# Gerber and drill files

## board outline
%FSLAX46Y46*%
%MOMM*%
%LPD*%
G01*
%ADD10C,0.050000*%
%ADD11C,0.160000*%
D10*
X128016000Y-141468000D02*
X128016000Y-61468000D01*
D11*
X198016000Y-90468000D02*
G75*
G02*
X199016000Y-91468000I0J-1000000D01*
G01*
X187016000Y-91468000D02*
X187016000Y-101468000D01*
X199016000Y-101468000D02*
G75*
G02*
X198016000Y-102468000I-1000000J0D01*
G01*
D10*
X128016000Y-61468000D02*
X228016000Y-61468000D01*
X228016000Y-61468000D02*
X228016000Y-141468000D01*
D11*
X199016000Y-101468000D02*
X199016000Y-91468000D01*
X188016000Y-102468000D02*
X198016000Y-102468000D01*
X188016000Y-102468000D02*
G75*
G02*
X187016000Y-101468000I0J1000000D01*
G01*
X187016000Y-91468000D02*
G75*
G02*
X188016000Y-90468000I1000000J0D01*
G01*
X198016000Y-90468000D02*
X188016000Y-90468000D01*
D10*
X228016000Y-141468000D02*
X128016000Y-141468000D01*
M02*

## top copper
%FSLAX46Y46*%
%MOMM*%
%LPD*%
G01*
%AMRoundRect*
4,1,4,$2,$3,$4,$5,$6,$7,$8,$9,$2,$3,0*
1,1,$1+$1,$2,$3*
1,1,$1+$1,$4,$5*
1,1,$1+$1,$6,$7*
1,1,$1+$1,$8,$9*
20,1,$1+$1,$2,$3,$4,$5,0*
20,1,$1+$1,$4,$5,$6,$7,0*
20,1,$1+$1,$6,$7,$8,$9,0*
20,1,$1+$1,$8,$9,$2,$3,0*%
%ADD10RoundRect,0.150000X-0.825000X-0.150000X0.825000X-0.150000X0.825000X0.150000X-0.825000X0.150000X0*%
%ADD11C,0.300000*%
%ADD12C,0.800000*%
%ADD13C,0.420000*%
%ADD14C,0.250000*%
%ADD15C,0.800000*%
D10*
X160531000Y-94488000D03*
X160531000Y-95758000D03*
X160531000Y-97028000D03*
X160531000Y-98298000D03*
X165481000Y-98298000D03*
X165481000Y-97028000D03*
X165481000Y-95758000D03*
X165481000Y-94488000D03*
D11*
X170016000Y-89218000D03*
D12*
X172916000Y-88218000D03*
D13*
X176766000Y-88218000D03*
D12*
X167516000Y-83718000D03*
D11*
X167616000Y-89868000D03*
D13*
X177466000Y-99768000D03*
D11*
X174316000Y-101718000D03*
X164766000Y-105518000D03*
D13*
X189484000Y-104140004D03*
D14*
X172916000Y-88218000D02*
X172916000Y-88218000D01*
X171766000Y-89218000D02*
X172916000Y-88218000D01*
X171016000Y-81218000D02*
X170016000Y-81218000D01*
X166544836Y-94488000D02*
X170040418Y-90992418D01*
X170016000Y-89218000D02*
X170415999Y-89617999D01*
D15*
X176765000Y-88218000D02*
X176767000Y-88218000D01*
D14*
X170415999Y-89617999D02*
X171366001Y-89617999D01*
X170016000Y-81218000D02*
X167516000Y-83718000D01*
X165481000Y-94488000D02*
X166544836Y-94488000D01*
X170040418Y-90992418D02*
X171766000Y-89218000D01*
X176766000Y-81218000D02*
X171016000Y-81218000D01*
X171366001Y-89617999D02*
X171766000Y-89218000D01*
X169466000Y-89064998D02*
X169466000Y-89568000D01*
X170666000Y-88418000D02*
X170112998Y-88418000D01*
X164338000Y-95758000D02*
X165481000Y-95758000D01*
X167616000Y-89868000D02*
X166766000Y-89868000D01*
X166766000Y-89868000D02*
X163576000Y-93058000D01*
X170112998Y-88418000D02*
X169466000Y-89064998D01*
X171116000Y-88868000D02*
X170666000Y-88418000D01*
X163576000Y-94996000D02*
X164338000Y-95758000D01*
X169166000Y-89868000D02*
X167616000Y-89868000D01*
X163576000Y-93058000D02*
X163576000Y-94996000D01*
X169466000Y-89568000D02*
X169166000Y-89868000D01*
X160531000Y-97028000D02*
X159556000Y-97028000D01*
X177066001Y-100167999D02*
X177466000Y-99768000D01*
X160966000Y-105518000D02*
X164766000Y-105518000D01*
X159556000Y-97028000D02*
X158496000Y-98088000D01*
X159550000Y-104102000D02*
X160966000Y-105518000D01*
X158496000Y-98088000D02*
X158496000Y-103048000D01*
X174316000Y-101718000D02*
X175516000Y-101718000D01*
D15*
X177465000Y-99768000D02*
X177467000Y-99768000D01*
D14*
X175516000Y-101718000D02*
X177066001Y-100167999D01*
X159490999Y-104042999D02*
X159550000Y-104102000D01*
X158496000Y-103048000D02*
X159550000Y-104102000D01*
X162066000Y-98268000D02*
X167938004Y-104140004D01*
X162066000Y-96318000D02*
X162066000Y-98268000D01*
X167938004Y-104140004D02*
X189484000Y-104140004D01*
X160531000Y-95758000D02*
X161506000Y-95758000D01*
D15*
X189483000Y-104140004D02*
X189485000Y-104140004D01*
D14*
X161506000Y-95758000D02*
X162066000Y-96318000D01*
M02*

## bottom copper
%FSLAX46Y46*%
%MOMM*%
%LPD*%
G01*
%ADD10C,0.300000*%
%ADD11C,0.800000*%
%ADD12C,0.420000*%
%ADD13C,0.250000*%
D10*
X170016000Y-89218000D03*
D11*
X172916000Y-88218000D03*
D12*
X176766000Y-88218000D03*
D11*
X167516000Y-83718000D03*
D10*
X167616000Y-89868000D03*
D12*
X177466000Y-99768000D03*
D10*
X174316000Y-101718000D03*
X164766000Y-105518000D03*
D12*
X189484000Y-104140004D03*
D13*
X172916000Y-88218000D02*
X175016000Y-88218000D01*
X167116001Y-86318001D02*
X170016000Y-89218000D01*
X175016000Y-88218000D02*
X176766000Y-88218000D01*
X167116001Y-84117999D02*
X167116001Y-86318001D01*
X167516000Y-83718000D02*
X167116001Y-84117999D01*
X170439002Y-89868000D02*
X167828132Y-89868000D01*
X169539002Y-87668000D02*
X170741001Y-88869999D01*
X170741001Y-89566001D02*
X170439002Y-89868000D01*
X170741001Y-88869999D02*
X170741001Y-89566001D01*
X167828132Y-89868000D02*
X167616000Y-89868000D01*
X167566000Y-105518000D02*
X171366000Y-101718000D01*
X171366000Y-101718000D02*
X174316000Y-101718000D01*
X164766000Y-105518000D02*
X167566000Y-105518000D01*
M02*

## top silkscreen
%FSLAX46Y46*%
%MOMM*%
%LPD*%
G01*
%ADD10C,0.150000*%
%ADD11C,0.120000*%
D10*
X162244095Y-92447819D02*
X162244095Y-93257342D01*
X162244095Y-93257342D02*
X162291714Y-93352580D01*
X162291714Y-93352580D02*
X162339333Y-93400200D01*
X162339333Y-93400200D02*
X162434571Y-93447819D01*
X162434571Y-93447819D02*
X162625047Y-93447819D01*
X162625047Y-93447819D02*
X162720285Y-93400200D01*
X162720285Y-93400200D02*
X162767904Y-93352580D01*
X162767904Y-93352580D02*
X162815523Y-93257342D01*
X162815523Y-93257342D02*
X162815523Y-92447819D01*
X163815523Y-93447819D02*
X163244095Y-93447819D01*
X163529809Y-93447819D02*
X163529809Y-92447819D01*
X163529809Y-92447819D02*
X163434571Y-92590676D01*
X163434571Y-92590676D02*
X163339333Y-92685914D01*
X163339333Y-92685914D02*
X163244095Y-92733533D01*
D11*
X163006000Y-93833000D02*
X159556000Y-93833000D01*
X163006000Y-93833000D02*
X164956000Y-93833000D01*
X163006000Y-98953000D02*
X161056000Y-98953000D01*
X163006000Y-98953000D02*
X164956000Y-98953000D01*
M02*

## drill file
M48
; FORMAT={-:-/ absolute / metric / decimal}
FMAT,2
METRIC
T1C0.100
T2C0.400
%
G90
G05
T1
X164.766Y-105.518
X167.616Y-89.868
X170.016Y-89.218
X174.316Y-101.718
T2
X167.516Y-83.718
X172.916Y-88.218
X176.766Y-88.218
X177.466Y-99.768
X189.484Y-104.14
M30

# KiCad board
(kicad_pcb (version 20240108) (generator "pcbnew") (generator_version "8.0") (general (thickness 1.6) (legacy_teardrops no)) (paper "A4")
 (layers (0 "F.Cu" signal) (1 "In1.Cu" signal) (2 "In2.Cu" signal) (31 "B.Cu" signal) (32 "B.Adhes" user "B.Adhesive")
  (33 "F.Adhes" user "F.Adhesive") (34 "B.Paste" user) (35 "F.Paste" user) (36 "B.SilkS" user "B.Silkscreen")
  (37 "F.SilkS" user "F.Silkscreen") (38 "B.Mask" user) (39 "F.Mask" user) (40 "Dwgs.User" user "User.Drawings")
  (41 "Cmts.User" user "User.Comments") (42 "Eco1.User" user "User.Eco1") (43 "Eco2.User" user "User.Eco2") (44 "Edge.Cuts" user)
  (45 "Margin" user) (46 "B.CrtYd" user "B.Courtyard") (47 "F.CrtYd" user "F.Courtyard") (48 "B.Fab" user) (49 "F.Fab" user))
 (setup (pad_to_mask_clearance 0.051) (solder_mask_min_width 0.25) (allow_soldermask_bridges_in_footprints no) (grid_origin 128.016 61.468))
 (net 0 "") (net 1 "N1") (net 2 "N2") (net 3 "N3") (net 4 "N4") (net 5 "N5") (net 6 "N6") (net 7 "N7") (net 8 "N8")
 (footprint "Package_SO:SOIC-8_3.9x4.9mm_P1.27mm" (layer "F.Cu") (at 163.006 96.393)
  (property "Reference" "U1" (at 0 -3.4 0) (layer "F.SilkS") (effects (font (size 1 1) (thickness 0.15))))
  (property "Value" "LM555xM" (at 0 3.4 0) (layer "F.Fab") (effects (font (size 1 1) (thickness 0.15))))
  (fp_line (start 0 -2.56) (end -3.45 -2.56) (stroke (width 0.12) (type solid)) (layer "F.SilkS"))
  (fp_line (start 0 -2.56) (end 1.95 -2.56) (stroke (width 0.12) (type solid)) (layer "F.SilkS"))
  (fp_line (start 0 2.56) (end -1.95 2.56) (stroke (width 0.12) (type solid)) (layer "F.SilkS"))
  (fp_line (start 0 2.56) (end 1.95 2.56) (stroke (width 0.12) (type solid)) (layer "F.SilkS"))
  (pad "1" smd roundrect (at -2.475 -1.905) (size 1.95 0.6) (layers "F.Cu" "F.Paste" "F.Mask") (roundrect_rratio 0.25) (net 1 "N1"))
  (pad "2" smd roundrect (at -2.475 -0.635) (size 1.95 0.6) (layers "F.Cu" "F.Paste" "F.Mask") (roundrect_rratio 0.25) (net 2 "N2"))
  (pad "3" smd roundrect (at -2.475 0.635) (size 1.95 0.6) (layers "F.Cu" "F.Paste" "F.Mask") (roundrect_rratio 0.25) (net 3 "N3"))
  (pad "4" smd roundrect (at -2.475 1.905) (size 1.95 0.6) (layers "F.Cu" "F.Paste" "F.Mask") (roundrect_rratio 0.25) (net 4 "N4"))
  (pad "5" smd roundrect (at 2.475 1.905) (size 1.95 0.6) (layers "F.Cu" "F.Paste" "F.Mask") (roundrect_rratio 0.25) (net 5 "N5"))
  (pad "6" smd roundrect (at 2.475 0.635) (size 1.95 0.6) (layers "F.Cu" "F.Paste" "F.Mask") (roundrect_rratio 0.25) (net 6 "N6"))
  (pad "7" smd roundrect (at 2.475 -0.635) (size 1.95 0.6) (layers "F.Cu" "F.Paste" "F.Mask") (roundrect_rratio 0.25) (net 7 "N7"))
  (pad "8" smd roundrect (at 2.475 -1.905) (size 1.95 0.6) (layers "F.Cu" "F.Paste" "F.Mask") (roundrect_rratio 0.25) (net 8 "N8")))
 (gr_line (start 128.016 141.468) (end 128.016 61.468) (stroke (width 0.05) (type solid)) (layer "Edge.Cuts"))
 (gr_arc (start 198.016 90.468) (mid 198.723107 90.760893) (end 199.016 91.468) (stroke (width 0.16) (type solid)) (layer "Edge.Cuts"))
 (gr_line (start 187.016 91.468) (end 187.016 101.468) (stroke (width 0.16) (type solid)) (layer "Edge.Cuts"))
 (gr_arc (start 199.016 101.468) (mid 198.723107 102.175107) (end 198.016 102.468) (stroke (width 0.16) (type solid)) (layer "Edge.Cuts"))
 (gr_line (start 128.016 61.468) (end 228.016 61.468) (stroke (width 0.05) (type solid)) (layer "Edge.Cuts"))
 (gr_line (start 228.016 61.468) (end 228.016 141.468) (stroke (width 0.05) (type solid)) (layer "Edge.Cuts"))
 (gr_line (start 199.016 101.468) (end 199.016 91.468) (stroke (width 0.16) (type solid)) (layer "Edge.Cuts"))
 (gr_line (start 188.016 102.468) (end 198.016 102.468) (stroke (width 0.16) (type solid)) (layer "Edge.Cuts"))
 (gr_arc (start 188.016 102.468) (mid 187.308893 102.175107) (end 187.016 101.468) (stroke (width 0.16) (type solid)) (layer "Edge.Cuts"))
 (gr_arc (start 187.016 91.468) (mid 187.308893 90.760893) (end 188.016 90.468) (stroke (width 0.16) (type solid)) (layer "Edge.Cuts"))
 (gr_line (start 198.016 90.468) (end 188.016 90.468) (stroke (width 0.16) (type solid)) (layer "Edge.Cuts"))
 (gr_line (start 228.016 141.468) (end 128.016 141.468) (stroke (width 0.05) (type solid)) (layer "Edge.Cuts"))
 (segment (start 172.916 88.218) (end 172.916 88.218) (width 0.25) (layer "F.Cu") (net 8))
 (segment (start 171.766 89.218) (end 172.916 88.218) (width 0.25) (layer "F.Cu") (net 8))
 (segment (start 171.016 81.218) (end 170.016 81.218) (width 0.25) (layer "F.Cu") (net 8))
 (segment (start 166.544836 94.488) (end 170.040418 90.992418) (width 0.25) (layer "F.Cu") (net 8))
 (segment (start 170.016 89.218) (end 170.415999 89.617999) (width 0.25) (layer "F.Cu") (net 8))
 (segment (start 176.765 88.218) (end 176.767 88.218) (width 0.8) (layer "F.Cu") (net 8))
 (segment (start 170.415999 89.617999) (end 171.366001 89.617999) (width 0.25) (layer "F.Cu") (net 8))
 (segment (start 170.016 81.218) (end 167.516 83.718) (width 0.25) (layer "F.Cu") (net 8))
 (segment (start 165.481 94.488) (end 166.544836 94.488) (width 0.25) (layer "F.Cu") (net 8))
 (segment (start 170.040418 90.992418) (end 171.766 89.218) (width 0.25) (layer "F.Cu") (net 8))
 (segment (start 176.766 81.218) (end 171.016 81.218) (width 0.25) (layer "F.Cu") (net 8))
 (segment (start 171.366001 89.617999) (end 171.766 89.218) (width 0.25) (layer "F.Cu") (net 8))
 (via (at 170.016 89.218) (size 0.3) (drill 0.1) (layers "F.Cu" "B.Cu") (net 8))
 (via (at 172.916 88.218) (size 0.8) (drill 0.4) (layers "F.Cu" "B.Cu") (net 8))
 (via (at 176.766 88.218) (size 0.42) (drill 0.4) (layers "F.Cu" "B.Cu") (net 8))
 (via (at 167.516 83.718) (size 0.8) (drill 0.4) (layers "F.Cu" "B.Cu") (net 8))
 (segment (start 172.916 88.218) (end 175.016 88.218) (width 0.25) (layer "B.Cu") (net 8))
 (segment (start 167.116001 86.318001) (end 170.016 89.218) (width 0.25) (layer "B.Cu") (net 8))
 (segment (start 175.016 88.218) (end 176.766 88.218) (width 0.25) (layer "B.Cu") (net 8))
 (segment (start 167.116001 84.117999) (end 167.116001 86.318001) (width 0.25) (layer "B.Cu") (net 8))
 (segment (start 167.516 83.718) (end 167.116001 84.117999) (width 0.25) (layer "B.Cu") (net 8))
 (segment (start 169.466 89.064998) (end 169.466 89.568) (width 0.25) (layer "F.Cu") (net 7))
 (segment (start 170.666 88.418) (end 170.112998 88.418) (width 0.25) (layer "F.Cu") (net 7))
 (segment (start 164.338 95.758) (end 165.481 95.758) (width 0.25) (layer "F.Cu") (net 7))
 (segment (start 167.616 89.868) (end 166.766 89.868) (width 0.25) (layer "F.Cu") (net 7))
 (segment (start 166.766 89.868) (end 163.576 93.058) (width 0.25) (layer "F.Cu") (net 7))
 (segment (start 170.112998 88.418) (end 169.466 89.064998) (width 0.25) (layer "F.Cu") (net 7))
 (segment (start 171.116 88.868) (end 170.666 88.418) (width 0.25) (layer "F.Cu") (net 7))
 (segment (start 163.576 94.996) (end 164.338 95.758) (width 0.25) (layer "F.Cu") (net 7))
 (segment (start 169.166 89.868) (end 167.616 89.868) (width 0.25) (layer "F.Cu") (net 7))
 (segment (start 163.576 93.058) (end 163.576 94.996) (width 0.25) (layer "F.Cu") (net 7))
 (segment (start 169.466 89.568) (end 169.166 89.868) (width 0.25) (layer "F.Cu") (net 7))
 (via (at 167.616 89.868) (size 0.3) (drill 0.1) (layers "F.Cu" "B.Cu") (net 7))
 (segment (start 170.439002 89.868) (end 167.828132 89.868) (width 0.25) (layer "B.Cu") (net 7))
 (segment (start 169.539002 87.668) (end 170.741001 88.869999) (width 0.25) (layer "B.Cu") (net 7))
 (segment (start 170.741001 89.566001) (end 170.439002 89.868) (width 0.25) (layer "B.Cu") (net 7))
 (segment (start 170.741001 88.869999) (end 170.741001 89.566001) (width 0.25) (layer "B.Cu") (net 7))
 (segment (start 167.828132 89.868) (end 167.616 89.868) (width 0.25) (layer "B.Cu") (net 7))
 (segment (start 160.531 97.028) (end 159.556 97.028) (width 0.25) (layer "F.Cu") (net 3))
 (segment (start 177.066001 100.167999) (end 177.466 99.768) (width 0.25) (layer "F.Cu") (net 3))
 (segment (start 160.966 105.518) (end 164.766 105.518) (width 0.25) (layer "F.Cu") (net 3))
 (segment (start 159.556 97.028) (end 158.496 98.088) (width 0.25) (layer "F.Cu") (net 3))
 (segment (start 159.55 104.102) (end 160.966 105.518) (width 0.25) (layer "F.Cu") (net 3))
 (segment (start 158.496 98.088) (end 158.496 103.048) (width 0.25) (layer "F.Cu") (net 3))
 (segment (start 174.316 101.718) (end 175.516 101.718) (width 0.25) (layer "F.Cu") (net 3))
 (segment (start 177.465 99.768) (end 177.467 99.768) (width 0.8) (layer "F.Cu") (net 3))
 (segment (start 175.516 101.718) (end 177.066001 100.167999) (width 0.25) (layer "F.Cu") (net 3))
 (segment (start 159.490999 104.042999) (end 159.55 104.102) (width 0.25) (layer "F.Cu") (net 3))
 (segment (start 158.496 103.048) (end 159.55 104.102) (width 0.25) (layer "F.Cu") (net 3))
 (via (at 177.466 99.768) (size 0.42) (drill 0.4) (layers "F.Cu" "B.Cu") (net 3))
 (via (at 174.316 101.718) (size 0.3) (drill 0.1) (layers "F.Cu" "B.Cu") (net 3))
 (via (at 164.766 105.518) (size 0.3) (drill 0.1) (layers "F.Cu" "B.Cu") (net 3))
 (segment (start 167.566 105.518) (end 171.366 101.718) (width 0.25) (layer "B.Cu") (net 3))
 (segment (start 171.366 101.718) (end 174.316 101.718) (width 0.25) (layer "B.Cu") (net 3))
 (segment (start 164.766 105.518) (end 167.566 105.518) (width 0.25) (layer "B.Cu") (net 3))
 (segment (start 162.066 98.268) (end 167.938004 104.140004) (width 0.25) (layer "F.Cu") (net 2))
 (segment (start 162.066 96.318) (end 162.066 98.268) (width 0.25) (layer "F.Cu") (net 2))
 (segment (start 167.938004 104.140004) (end 189.484 104.140004) (width 0.25) (layer "F.Cu") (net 2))
 (segment (start 160.531 95.758) (end 161.506 95.758) (width 0.25) (layer "F.Cu") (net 2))
 (segment (start 189.483 104.140004) (end 189.485 104.140004) (width 0.8) (layer "F.Cu") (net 2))
 (segment (start 161.506 95.758) (end 162.066 96.318) (width 0.25) (layer "F.Cu") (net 2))
 (via (at 189.484 104.140004) (size 0.42) (drill 0.4) (layers "F.Cu" "B.Cu") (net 2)))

